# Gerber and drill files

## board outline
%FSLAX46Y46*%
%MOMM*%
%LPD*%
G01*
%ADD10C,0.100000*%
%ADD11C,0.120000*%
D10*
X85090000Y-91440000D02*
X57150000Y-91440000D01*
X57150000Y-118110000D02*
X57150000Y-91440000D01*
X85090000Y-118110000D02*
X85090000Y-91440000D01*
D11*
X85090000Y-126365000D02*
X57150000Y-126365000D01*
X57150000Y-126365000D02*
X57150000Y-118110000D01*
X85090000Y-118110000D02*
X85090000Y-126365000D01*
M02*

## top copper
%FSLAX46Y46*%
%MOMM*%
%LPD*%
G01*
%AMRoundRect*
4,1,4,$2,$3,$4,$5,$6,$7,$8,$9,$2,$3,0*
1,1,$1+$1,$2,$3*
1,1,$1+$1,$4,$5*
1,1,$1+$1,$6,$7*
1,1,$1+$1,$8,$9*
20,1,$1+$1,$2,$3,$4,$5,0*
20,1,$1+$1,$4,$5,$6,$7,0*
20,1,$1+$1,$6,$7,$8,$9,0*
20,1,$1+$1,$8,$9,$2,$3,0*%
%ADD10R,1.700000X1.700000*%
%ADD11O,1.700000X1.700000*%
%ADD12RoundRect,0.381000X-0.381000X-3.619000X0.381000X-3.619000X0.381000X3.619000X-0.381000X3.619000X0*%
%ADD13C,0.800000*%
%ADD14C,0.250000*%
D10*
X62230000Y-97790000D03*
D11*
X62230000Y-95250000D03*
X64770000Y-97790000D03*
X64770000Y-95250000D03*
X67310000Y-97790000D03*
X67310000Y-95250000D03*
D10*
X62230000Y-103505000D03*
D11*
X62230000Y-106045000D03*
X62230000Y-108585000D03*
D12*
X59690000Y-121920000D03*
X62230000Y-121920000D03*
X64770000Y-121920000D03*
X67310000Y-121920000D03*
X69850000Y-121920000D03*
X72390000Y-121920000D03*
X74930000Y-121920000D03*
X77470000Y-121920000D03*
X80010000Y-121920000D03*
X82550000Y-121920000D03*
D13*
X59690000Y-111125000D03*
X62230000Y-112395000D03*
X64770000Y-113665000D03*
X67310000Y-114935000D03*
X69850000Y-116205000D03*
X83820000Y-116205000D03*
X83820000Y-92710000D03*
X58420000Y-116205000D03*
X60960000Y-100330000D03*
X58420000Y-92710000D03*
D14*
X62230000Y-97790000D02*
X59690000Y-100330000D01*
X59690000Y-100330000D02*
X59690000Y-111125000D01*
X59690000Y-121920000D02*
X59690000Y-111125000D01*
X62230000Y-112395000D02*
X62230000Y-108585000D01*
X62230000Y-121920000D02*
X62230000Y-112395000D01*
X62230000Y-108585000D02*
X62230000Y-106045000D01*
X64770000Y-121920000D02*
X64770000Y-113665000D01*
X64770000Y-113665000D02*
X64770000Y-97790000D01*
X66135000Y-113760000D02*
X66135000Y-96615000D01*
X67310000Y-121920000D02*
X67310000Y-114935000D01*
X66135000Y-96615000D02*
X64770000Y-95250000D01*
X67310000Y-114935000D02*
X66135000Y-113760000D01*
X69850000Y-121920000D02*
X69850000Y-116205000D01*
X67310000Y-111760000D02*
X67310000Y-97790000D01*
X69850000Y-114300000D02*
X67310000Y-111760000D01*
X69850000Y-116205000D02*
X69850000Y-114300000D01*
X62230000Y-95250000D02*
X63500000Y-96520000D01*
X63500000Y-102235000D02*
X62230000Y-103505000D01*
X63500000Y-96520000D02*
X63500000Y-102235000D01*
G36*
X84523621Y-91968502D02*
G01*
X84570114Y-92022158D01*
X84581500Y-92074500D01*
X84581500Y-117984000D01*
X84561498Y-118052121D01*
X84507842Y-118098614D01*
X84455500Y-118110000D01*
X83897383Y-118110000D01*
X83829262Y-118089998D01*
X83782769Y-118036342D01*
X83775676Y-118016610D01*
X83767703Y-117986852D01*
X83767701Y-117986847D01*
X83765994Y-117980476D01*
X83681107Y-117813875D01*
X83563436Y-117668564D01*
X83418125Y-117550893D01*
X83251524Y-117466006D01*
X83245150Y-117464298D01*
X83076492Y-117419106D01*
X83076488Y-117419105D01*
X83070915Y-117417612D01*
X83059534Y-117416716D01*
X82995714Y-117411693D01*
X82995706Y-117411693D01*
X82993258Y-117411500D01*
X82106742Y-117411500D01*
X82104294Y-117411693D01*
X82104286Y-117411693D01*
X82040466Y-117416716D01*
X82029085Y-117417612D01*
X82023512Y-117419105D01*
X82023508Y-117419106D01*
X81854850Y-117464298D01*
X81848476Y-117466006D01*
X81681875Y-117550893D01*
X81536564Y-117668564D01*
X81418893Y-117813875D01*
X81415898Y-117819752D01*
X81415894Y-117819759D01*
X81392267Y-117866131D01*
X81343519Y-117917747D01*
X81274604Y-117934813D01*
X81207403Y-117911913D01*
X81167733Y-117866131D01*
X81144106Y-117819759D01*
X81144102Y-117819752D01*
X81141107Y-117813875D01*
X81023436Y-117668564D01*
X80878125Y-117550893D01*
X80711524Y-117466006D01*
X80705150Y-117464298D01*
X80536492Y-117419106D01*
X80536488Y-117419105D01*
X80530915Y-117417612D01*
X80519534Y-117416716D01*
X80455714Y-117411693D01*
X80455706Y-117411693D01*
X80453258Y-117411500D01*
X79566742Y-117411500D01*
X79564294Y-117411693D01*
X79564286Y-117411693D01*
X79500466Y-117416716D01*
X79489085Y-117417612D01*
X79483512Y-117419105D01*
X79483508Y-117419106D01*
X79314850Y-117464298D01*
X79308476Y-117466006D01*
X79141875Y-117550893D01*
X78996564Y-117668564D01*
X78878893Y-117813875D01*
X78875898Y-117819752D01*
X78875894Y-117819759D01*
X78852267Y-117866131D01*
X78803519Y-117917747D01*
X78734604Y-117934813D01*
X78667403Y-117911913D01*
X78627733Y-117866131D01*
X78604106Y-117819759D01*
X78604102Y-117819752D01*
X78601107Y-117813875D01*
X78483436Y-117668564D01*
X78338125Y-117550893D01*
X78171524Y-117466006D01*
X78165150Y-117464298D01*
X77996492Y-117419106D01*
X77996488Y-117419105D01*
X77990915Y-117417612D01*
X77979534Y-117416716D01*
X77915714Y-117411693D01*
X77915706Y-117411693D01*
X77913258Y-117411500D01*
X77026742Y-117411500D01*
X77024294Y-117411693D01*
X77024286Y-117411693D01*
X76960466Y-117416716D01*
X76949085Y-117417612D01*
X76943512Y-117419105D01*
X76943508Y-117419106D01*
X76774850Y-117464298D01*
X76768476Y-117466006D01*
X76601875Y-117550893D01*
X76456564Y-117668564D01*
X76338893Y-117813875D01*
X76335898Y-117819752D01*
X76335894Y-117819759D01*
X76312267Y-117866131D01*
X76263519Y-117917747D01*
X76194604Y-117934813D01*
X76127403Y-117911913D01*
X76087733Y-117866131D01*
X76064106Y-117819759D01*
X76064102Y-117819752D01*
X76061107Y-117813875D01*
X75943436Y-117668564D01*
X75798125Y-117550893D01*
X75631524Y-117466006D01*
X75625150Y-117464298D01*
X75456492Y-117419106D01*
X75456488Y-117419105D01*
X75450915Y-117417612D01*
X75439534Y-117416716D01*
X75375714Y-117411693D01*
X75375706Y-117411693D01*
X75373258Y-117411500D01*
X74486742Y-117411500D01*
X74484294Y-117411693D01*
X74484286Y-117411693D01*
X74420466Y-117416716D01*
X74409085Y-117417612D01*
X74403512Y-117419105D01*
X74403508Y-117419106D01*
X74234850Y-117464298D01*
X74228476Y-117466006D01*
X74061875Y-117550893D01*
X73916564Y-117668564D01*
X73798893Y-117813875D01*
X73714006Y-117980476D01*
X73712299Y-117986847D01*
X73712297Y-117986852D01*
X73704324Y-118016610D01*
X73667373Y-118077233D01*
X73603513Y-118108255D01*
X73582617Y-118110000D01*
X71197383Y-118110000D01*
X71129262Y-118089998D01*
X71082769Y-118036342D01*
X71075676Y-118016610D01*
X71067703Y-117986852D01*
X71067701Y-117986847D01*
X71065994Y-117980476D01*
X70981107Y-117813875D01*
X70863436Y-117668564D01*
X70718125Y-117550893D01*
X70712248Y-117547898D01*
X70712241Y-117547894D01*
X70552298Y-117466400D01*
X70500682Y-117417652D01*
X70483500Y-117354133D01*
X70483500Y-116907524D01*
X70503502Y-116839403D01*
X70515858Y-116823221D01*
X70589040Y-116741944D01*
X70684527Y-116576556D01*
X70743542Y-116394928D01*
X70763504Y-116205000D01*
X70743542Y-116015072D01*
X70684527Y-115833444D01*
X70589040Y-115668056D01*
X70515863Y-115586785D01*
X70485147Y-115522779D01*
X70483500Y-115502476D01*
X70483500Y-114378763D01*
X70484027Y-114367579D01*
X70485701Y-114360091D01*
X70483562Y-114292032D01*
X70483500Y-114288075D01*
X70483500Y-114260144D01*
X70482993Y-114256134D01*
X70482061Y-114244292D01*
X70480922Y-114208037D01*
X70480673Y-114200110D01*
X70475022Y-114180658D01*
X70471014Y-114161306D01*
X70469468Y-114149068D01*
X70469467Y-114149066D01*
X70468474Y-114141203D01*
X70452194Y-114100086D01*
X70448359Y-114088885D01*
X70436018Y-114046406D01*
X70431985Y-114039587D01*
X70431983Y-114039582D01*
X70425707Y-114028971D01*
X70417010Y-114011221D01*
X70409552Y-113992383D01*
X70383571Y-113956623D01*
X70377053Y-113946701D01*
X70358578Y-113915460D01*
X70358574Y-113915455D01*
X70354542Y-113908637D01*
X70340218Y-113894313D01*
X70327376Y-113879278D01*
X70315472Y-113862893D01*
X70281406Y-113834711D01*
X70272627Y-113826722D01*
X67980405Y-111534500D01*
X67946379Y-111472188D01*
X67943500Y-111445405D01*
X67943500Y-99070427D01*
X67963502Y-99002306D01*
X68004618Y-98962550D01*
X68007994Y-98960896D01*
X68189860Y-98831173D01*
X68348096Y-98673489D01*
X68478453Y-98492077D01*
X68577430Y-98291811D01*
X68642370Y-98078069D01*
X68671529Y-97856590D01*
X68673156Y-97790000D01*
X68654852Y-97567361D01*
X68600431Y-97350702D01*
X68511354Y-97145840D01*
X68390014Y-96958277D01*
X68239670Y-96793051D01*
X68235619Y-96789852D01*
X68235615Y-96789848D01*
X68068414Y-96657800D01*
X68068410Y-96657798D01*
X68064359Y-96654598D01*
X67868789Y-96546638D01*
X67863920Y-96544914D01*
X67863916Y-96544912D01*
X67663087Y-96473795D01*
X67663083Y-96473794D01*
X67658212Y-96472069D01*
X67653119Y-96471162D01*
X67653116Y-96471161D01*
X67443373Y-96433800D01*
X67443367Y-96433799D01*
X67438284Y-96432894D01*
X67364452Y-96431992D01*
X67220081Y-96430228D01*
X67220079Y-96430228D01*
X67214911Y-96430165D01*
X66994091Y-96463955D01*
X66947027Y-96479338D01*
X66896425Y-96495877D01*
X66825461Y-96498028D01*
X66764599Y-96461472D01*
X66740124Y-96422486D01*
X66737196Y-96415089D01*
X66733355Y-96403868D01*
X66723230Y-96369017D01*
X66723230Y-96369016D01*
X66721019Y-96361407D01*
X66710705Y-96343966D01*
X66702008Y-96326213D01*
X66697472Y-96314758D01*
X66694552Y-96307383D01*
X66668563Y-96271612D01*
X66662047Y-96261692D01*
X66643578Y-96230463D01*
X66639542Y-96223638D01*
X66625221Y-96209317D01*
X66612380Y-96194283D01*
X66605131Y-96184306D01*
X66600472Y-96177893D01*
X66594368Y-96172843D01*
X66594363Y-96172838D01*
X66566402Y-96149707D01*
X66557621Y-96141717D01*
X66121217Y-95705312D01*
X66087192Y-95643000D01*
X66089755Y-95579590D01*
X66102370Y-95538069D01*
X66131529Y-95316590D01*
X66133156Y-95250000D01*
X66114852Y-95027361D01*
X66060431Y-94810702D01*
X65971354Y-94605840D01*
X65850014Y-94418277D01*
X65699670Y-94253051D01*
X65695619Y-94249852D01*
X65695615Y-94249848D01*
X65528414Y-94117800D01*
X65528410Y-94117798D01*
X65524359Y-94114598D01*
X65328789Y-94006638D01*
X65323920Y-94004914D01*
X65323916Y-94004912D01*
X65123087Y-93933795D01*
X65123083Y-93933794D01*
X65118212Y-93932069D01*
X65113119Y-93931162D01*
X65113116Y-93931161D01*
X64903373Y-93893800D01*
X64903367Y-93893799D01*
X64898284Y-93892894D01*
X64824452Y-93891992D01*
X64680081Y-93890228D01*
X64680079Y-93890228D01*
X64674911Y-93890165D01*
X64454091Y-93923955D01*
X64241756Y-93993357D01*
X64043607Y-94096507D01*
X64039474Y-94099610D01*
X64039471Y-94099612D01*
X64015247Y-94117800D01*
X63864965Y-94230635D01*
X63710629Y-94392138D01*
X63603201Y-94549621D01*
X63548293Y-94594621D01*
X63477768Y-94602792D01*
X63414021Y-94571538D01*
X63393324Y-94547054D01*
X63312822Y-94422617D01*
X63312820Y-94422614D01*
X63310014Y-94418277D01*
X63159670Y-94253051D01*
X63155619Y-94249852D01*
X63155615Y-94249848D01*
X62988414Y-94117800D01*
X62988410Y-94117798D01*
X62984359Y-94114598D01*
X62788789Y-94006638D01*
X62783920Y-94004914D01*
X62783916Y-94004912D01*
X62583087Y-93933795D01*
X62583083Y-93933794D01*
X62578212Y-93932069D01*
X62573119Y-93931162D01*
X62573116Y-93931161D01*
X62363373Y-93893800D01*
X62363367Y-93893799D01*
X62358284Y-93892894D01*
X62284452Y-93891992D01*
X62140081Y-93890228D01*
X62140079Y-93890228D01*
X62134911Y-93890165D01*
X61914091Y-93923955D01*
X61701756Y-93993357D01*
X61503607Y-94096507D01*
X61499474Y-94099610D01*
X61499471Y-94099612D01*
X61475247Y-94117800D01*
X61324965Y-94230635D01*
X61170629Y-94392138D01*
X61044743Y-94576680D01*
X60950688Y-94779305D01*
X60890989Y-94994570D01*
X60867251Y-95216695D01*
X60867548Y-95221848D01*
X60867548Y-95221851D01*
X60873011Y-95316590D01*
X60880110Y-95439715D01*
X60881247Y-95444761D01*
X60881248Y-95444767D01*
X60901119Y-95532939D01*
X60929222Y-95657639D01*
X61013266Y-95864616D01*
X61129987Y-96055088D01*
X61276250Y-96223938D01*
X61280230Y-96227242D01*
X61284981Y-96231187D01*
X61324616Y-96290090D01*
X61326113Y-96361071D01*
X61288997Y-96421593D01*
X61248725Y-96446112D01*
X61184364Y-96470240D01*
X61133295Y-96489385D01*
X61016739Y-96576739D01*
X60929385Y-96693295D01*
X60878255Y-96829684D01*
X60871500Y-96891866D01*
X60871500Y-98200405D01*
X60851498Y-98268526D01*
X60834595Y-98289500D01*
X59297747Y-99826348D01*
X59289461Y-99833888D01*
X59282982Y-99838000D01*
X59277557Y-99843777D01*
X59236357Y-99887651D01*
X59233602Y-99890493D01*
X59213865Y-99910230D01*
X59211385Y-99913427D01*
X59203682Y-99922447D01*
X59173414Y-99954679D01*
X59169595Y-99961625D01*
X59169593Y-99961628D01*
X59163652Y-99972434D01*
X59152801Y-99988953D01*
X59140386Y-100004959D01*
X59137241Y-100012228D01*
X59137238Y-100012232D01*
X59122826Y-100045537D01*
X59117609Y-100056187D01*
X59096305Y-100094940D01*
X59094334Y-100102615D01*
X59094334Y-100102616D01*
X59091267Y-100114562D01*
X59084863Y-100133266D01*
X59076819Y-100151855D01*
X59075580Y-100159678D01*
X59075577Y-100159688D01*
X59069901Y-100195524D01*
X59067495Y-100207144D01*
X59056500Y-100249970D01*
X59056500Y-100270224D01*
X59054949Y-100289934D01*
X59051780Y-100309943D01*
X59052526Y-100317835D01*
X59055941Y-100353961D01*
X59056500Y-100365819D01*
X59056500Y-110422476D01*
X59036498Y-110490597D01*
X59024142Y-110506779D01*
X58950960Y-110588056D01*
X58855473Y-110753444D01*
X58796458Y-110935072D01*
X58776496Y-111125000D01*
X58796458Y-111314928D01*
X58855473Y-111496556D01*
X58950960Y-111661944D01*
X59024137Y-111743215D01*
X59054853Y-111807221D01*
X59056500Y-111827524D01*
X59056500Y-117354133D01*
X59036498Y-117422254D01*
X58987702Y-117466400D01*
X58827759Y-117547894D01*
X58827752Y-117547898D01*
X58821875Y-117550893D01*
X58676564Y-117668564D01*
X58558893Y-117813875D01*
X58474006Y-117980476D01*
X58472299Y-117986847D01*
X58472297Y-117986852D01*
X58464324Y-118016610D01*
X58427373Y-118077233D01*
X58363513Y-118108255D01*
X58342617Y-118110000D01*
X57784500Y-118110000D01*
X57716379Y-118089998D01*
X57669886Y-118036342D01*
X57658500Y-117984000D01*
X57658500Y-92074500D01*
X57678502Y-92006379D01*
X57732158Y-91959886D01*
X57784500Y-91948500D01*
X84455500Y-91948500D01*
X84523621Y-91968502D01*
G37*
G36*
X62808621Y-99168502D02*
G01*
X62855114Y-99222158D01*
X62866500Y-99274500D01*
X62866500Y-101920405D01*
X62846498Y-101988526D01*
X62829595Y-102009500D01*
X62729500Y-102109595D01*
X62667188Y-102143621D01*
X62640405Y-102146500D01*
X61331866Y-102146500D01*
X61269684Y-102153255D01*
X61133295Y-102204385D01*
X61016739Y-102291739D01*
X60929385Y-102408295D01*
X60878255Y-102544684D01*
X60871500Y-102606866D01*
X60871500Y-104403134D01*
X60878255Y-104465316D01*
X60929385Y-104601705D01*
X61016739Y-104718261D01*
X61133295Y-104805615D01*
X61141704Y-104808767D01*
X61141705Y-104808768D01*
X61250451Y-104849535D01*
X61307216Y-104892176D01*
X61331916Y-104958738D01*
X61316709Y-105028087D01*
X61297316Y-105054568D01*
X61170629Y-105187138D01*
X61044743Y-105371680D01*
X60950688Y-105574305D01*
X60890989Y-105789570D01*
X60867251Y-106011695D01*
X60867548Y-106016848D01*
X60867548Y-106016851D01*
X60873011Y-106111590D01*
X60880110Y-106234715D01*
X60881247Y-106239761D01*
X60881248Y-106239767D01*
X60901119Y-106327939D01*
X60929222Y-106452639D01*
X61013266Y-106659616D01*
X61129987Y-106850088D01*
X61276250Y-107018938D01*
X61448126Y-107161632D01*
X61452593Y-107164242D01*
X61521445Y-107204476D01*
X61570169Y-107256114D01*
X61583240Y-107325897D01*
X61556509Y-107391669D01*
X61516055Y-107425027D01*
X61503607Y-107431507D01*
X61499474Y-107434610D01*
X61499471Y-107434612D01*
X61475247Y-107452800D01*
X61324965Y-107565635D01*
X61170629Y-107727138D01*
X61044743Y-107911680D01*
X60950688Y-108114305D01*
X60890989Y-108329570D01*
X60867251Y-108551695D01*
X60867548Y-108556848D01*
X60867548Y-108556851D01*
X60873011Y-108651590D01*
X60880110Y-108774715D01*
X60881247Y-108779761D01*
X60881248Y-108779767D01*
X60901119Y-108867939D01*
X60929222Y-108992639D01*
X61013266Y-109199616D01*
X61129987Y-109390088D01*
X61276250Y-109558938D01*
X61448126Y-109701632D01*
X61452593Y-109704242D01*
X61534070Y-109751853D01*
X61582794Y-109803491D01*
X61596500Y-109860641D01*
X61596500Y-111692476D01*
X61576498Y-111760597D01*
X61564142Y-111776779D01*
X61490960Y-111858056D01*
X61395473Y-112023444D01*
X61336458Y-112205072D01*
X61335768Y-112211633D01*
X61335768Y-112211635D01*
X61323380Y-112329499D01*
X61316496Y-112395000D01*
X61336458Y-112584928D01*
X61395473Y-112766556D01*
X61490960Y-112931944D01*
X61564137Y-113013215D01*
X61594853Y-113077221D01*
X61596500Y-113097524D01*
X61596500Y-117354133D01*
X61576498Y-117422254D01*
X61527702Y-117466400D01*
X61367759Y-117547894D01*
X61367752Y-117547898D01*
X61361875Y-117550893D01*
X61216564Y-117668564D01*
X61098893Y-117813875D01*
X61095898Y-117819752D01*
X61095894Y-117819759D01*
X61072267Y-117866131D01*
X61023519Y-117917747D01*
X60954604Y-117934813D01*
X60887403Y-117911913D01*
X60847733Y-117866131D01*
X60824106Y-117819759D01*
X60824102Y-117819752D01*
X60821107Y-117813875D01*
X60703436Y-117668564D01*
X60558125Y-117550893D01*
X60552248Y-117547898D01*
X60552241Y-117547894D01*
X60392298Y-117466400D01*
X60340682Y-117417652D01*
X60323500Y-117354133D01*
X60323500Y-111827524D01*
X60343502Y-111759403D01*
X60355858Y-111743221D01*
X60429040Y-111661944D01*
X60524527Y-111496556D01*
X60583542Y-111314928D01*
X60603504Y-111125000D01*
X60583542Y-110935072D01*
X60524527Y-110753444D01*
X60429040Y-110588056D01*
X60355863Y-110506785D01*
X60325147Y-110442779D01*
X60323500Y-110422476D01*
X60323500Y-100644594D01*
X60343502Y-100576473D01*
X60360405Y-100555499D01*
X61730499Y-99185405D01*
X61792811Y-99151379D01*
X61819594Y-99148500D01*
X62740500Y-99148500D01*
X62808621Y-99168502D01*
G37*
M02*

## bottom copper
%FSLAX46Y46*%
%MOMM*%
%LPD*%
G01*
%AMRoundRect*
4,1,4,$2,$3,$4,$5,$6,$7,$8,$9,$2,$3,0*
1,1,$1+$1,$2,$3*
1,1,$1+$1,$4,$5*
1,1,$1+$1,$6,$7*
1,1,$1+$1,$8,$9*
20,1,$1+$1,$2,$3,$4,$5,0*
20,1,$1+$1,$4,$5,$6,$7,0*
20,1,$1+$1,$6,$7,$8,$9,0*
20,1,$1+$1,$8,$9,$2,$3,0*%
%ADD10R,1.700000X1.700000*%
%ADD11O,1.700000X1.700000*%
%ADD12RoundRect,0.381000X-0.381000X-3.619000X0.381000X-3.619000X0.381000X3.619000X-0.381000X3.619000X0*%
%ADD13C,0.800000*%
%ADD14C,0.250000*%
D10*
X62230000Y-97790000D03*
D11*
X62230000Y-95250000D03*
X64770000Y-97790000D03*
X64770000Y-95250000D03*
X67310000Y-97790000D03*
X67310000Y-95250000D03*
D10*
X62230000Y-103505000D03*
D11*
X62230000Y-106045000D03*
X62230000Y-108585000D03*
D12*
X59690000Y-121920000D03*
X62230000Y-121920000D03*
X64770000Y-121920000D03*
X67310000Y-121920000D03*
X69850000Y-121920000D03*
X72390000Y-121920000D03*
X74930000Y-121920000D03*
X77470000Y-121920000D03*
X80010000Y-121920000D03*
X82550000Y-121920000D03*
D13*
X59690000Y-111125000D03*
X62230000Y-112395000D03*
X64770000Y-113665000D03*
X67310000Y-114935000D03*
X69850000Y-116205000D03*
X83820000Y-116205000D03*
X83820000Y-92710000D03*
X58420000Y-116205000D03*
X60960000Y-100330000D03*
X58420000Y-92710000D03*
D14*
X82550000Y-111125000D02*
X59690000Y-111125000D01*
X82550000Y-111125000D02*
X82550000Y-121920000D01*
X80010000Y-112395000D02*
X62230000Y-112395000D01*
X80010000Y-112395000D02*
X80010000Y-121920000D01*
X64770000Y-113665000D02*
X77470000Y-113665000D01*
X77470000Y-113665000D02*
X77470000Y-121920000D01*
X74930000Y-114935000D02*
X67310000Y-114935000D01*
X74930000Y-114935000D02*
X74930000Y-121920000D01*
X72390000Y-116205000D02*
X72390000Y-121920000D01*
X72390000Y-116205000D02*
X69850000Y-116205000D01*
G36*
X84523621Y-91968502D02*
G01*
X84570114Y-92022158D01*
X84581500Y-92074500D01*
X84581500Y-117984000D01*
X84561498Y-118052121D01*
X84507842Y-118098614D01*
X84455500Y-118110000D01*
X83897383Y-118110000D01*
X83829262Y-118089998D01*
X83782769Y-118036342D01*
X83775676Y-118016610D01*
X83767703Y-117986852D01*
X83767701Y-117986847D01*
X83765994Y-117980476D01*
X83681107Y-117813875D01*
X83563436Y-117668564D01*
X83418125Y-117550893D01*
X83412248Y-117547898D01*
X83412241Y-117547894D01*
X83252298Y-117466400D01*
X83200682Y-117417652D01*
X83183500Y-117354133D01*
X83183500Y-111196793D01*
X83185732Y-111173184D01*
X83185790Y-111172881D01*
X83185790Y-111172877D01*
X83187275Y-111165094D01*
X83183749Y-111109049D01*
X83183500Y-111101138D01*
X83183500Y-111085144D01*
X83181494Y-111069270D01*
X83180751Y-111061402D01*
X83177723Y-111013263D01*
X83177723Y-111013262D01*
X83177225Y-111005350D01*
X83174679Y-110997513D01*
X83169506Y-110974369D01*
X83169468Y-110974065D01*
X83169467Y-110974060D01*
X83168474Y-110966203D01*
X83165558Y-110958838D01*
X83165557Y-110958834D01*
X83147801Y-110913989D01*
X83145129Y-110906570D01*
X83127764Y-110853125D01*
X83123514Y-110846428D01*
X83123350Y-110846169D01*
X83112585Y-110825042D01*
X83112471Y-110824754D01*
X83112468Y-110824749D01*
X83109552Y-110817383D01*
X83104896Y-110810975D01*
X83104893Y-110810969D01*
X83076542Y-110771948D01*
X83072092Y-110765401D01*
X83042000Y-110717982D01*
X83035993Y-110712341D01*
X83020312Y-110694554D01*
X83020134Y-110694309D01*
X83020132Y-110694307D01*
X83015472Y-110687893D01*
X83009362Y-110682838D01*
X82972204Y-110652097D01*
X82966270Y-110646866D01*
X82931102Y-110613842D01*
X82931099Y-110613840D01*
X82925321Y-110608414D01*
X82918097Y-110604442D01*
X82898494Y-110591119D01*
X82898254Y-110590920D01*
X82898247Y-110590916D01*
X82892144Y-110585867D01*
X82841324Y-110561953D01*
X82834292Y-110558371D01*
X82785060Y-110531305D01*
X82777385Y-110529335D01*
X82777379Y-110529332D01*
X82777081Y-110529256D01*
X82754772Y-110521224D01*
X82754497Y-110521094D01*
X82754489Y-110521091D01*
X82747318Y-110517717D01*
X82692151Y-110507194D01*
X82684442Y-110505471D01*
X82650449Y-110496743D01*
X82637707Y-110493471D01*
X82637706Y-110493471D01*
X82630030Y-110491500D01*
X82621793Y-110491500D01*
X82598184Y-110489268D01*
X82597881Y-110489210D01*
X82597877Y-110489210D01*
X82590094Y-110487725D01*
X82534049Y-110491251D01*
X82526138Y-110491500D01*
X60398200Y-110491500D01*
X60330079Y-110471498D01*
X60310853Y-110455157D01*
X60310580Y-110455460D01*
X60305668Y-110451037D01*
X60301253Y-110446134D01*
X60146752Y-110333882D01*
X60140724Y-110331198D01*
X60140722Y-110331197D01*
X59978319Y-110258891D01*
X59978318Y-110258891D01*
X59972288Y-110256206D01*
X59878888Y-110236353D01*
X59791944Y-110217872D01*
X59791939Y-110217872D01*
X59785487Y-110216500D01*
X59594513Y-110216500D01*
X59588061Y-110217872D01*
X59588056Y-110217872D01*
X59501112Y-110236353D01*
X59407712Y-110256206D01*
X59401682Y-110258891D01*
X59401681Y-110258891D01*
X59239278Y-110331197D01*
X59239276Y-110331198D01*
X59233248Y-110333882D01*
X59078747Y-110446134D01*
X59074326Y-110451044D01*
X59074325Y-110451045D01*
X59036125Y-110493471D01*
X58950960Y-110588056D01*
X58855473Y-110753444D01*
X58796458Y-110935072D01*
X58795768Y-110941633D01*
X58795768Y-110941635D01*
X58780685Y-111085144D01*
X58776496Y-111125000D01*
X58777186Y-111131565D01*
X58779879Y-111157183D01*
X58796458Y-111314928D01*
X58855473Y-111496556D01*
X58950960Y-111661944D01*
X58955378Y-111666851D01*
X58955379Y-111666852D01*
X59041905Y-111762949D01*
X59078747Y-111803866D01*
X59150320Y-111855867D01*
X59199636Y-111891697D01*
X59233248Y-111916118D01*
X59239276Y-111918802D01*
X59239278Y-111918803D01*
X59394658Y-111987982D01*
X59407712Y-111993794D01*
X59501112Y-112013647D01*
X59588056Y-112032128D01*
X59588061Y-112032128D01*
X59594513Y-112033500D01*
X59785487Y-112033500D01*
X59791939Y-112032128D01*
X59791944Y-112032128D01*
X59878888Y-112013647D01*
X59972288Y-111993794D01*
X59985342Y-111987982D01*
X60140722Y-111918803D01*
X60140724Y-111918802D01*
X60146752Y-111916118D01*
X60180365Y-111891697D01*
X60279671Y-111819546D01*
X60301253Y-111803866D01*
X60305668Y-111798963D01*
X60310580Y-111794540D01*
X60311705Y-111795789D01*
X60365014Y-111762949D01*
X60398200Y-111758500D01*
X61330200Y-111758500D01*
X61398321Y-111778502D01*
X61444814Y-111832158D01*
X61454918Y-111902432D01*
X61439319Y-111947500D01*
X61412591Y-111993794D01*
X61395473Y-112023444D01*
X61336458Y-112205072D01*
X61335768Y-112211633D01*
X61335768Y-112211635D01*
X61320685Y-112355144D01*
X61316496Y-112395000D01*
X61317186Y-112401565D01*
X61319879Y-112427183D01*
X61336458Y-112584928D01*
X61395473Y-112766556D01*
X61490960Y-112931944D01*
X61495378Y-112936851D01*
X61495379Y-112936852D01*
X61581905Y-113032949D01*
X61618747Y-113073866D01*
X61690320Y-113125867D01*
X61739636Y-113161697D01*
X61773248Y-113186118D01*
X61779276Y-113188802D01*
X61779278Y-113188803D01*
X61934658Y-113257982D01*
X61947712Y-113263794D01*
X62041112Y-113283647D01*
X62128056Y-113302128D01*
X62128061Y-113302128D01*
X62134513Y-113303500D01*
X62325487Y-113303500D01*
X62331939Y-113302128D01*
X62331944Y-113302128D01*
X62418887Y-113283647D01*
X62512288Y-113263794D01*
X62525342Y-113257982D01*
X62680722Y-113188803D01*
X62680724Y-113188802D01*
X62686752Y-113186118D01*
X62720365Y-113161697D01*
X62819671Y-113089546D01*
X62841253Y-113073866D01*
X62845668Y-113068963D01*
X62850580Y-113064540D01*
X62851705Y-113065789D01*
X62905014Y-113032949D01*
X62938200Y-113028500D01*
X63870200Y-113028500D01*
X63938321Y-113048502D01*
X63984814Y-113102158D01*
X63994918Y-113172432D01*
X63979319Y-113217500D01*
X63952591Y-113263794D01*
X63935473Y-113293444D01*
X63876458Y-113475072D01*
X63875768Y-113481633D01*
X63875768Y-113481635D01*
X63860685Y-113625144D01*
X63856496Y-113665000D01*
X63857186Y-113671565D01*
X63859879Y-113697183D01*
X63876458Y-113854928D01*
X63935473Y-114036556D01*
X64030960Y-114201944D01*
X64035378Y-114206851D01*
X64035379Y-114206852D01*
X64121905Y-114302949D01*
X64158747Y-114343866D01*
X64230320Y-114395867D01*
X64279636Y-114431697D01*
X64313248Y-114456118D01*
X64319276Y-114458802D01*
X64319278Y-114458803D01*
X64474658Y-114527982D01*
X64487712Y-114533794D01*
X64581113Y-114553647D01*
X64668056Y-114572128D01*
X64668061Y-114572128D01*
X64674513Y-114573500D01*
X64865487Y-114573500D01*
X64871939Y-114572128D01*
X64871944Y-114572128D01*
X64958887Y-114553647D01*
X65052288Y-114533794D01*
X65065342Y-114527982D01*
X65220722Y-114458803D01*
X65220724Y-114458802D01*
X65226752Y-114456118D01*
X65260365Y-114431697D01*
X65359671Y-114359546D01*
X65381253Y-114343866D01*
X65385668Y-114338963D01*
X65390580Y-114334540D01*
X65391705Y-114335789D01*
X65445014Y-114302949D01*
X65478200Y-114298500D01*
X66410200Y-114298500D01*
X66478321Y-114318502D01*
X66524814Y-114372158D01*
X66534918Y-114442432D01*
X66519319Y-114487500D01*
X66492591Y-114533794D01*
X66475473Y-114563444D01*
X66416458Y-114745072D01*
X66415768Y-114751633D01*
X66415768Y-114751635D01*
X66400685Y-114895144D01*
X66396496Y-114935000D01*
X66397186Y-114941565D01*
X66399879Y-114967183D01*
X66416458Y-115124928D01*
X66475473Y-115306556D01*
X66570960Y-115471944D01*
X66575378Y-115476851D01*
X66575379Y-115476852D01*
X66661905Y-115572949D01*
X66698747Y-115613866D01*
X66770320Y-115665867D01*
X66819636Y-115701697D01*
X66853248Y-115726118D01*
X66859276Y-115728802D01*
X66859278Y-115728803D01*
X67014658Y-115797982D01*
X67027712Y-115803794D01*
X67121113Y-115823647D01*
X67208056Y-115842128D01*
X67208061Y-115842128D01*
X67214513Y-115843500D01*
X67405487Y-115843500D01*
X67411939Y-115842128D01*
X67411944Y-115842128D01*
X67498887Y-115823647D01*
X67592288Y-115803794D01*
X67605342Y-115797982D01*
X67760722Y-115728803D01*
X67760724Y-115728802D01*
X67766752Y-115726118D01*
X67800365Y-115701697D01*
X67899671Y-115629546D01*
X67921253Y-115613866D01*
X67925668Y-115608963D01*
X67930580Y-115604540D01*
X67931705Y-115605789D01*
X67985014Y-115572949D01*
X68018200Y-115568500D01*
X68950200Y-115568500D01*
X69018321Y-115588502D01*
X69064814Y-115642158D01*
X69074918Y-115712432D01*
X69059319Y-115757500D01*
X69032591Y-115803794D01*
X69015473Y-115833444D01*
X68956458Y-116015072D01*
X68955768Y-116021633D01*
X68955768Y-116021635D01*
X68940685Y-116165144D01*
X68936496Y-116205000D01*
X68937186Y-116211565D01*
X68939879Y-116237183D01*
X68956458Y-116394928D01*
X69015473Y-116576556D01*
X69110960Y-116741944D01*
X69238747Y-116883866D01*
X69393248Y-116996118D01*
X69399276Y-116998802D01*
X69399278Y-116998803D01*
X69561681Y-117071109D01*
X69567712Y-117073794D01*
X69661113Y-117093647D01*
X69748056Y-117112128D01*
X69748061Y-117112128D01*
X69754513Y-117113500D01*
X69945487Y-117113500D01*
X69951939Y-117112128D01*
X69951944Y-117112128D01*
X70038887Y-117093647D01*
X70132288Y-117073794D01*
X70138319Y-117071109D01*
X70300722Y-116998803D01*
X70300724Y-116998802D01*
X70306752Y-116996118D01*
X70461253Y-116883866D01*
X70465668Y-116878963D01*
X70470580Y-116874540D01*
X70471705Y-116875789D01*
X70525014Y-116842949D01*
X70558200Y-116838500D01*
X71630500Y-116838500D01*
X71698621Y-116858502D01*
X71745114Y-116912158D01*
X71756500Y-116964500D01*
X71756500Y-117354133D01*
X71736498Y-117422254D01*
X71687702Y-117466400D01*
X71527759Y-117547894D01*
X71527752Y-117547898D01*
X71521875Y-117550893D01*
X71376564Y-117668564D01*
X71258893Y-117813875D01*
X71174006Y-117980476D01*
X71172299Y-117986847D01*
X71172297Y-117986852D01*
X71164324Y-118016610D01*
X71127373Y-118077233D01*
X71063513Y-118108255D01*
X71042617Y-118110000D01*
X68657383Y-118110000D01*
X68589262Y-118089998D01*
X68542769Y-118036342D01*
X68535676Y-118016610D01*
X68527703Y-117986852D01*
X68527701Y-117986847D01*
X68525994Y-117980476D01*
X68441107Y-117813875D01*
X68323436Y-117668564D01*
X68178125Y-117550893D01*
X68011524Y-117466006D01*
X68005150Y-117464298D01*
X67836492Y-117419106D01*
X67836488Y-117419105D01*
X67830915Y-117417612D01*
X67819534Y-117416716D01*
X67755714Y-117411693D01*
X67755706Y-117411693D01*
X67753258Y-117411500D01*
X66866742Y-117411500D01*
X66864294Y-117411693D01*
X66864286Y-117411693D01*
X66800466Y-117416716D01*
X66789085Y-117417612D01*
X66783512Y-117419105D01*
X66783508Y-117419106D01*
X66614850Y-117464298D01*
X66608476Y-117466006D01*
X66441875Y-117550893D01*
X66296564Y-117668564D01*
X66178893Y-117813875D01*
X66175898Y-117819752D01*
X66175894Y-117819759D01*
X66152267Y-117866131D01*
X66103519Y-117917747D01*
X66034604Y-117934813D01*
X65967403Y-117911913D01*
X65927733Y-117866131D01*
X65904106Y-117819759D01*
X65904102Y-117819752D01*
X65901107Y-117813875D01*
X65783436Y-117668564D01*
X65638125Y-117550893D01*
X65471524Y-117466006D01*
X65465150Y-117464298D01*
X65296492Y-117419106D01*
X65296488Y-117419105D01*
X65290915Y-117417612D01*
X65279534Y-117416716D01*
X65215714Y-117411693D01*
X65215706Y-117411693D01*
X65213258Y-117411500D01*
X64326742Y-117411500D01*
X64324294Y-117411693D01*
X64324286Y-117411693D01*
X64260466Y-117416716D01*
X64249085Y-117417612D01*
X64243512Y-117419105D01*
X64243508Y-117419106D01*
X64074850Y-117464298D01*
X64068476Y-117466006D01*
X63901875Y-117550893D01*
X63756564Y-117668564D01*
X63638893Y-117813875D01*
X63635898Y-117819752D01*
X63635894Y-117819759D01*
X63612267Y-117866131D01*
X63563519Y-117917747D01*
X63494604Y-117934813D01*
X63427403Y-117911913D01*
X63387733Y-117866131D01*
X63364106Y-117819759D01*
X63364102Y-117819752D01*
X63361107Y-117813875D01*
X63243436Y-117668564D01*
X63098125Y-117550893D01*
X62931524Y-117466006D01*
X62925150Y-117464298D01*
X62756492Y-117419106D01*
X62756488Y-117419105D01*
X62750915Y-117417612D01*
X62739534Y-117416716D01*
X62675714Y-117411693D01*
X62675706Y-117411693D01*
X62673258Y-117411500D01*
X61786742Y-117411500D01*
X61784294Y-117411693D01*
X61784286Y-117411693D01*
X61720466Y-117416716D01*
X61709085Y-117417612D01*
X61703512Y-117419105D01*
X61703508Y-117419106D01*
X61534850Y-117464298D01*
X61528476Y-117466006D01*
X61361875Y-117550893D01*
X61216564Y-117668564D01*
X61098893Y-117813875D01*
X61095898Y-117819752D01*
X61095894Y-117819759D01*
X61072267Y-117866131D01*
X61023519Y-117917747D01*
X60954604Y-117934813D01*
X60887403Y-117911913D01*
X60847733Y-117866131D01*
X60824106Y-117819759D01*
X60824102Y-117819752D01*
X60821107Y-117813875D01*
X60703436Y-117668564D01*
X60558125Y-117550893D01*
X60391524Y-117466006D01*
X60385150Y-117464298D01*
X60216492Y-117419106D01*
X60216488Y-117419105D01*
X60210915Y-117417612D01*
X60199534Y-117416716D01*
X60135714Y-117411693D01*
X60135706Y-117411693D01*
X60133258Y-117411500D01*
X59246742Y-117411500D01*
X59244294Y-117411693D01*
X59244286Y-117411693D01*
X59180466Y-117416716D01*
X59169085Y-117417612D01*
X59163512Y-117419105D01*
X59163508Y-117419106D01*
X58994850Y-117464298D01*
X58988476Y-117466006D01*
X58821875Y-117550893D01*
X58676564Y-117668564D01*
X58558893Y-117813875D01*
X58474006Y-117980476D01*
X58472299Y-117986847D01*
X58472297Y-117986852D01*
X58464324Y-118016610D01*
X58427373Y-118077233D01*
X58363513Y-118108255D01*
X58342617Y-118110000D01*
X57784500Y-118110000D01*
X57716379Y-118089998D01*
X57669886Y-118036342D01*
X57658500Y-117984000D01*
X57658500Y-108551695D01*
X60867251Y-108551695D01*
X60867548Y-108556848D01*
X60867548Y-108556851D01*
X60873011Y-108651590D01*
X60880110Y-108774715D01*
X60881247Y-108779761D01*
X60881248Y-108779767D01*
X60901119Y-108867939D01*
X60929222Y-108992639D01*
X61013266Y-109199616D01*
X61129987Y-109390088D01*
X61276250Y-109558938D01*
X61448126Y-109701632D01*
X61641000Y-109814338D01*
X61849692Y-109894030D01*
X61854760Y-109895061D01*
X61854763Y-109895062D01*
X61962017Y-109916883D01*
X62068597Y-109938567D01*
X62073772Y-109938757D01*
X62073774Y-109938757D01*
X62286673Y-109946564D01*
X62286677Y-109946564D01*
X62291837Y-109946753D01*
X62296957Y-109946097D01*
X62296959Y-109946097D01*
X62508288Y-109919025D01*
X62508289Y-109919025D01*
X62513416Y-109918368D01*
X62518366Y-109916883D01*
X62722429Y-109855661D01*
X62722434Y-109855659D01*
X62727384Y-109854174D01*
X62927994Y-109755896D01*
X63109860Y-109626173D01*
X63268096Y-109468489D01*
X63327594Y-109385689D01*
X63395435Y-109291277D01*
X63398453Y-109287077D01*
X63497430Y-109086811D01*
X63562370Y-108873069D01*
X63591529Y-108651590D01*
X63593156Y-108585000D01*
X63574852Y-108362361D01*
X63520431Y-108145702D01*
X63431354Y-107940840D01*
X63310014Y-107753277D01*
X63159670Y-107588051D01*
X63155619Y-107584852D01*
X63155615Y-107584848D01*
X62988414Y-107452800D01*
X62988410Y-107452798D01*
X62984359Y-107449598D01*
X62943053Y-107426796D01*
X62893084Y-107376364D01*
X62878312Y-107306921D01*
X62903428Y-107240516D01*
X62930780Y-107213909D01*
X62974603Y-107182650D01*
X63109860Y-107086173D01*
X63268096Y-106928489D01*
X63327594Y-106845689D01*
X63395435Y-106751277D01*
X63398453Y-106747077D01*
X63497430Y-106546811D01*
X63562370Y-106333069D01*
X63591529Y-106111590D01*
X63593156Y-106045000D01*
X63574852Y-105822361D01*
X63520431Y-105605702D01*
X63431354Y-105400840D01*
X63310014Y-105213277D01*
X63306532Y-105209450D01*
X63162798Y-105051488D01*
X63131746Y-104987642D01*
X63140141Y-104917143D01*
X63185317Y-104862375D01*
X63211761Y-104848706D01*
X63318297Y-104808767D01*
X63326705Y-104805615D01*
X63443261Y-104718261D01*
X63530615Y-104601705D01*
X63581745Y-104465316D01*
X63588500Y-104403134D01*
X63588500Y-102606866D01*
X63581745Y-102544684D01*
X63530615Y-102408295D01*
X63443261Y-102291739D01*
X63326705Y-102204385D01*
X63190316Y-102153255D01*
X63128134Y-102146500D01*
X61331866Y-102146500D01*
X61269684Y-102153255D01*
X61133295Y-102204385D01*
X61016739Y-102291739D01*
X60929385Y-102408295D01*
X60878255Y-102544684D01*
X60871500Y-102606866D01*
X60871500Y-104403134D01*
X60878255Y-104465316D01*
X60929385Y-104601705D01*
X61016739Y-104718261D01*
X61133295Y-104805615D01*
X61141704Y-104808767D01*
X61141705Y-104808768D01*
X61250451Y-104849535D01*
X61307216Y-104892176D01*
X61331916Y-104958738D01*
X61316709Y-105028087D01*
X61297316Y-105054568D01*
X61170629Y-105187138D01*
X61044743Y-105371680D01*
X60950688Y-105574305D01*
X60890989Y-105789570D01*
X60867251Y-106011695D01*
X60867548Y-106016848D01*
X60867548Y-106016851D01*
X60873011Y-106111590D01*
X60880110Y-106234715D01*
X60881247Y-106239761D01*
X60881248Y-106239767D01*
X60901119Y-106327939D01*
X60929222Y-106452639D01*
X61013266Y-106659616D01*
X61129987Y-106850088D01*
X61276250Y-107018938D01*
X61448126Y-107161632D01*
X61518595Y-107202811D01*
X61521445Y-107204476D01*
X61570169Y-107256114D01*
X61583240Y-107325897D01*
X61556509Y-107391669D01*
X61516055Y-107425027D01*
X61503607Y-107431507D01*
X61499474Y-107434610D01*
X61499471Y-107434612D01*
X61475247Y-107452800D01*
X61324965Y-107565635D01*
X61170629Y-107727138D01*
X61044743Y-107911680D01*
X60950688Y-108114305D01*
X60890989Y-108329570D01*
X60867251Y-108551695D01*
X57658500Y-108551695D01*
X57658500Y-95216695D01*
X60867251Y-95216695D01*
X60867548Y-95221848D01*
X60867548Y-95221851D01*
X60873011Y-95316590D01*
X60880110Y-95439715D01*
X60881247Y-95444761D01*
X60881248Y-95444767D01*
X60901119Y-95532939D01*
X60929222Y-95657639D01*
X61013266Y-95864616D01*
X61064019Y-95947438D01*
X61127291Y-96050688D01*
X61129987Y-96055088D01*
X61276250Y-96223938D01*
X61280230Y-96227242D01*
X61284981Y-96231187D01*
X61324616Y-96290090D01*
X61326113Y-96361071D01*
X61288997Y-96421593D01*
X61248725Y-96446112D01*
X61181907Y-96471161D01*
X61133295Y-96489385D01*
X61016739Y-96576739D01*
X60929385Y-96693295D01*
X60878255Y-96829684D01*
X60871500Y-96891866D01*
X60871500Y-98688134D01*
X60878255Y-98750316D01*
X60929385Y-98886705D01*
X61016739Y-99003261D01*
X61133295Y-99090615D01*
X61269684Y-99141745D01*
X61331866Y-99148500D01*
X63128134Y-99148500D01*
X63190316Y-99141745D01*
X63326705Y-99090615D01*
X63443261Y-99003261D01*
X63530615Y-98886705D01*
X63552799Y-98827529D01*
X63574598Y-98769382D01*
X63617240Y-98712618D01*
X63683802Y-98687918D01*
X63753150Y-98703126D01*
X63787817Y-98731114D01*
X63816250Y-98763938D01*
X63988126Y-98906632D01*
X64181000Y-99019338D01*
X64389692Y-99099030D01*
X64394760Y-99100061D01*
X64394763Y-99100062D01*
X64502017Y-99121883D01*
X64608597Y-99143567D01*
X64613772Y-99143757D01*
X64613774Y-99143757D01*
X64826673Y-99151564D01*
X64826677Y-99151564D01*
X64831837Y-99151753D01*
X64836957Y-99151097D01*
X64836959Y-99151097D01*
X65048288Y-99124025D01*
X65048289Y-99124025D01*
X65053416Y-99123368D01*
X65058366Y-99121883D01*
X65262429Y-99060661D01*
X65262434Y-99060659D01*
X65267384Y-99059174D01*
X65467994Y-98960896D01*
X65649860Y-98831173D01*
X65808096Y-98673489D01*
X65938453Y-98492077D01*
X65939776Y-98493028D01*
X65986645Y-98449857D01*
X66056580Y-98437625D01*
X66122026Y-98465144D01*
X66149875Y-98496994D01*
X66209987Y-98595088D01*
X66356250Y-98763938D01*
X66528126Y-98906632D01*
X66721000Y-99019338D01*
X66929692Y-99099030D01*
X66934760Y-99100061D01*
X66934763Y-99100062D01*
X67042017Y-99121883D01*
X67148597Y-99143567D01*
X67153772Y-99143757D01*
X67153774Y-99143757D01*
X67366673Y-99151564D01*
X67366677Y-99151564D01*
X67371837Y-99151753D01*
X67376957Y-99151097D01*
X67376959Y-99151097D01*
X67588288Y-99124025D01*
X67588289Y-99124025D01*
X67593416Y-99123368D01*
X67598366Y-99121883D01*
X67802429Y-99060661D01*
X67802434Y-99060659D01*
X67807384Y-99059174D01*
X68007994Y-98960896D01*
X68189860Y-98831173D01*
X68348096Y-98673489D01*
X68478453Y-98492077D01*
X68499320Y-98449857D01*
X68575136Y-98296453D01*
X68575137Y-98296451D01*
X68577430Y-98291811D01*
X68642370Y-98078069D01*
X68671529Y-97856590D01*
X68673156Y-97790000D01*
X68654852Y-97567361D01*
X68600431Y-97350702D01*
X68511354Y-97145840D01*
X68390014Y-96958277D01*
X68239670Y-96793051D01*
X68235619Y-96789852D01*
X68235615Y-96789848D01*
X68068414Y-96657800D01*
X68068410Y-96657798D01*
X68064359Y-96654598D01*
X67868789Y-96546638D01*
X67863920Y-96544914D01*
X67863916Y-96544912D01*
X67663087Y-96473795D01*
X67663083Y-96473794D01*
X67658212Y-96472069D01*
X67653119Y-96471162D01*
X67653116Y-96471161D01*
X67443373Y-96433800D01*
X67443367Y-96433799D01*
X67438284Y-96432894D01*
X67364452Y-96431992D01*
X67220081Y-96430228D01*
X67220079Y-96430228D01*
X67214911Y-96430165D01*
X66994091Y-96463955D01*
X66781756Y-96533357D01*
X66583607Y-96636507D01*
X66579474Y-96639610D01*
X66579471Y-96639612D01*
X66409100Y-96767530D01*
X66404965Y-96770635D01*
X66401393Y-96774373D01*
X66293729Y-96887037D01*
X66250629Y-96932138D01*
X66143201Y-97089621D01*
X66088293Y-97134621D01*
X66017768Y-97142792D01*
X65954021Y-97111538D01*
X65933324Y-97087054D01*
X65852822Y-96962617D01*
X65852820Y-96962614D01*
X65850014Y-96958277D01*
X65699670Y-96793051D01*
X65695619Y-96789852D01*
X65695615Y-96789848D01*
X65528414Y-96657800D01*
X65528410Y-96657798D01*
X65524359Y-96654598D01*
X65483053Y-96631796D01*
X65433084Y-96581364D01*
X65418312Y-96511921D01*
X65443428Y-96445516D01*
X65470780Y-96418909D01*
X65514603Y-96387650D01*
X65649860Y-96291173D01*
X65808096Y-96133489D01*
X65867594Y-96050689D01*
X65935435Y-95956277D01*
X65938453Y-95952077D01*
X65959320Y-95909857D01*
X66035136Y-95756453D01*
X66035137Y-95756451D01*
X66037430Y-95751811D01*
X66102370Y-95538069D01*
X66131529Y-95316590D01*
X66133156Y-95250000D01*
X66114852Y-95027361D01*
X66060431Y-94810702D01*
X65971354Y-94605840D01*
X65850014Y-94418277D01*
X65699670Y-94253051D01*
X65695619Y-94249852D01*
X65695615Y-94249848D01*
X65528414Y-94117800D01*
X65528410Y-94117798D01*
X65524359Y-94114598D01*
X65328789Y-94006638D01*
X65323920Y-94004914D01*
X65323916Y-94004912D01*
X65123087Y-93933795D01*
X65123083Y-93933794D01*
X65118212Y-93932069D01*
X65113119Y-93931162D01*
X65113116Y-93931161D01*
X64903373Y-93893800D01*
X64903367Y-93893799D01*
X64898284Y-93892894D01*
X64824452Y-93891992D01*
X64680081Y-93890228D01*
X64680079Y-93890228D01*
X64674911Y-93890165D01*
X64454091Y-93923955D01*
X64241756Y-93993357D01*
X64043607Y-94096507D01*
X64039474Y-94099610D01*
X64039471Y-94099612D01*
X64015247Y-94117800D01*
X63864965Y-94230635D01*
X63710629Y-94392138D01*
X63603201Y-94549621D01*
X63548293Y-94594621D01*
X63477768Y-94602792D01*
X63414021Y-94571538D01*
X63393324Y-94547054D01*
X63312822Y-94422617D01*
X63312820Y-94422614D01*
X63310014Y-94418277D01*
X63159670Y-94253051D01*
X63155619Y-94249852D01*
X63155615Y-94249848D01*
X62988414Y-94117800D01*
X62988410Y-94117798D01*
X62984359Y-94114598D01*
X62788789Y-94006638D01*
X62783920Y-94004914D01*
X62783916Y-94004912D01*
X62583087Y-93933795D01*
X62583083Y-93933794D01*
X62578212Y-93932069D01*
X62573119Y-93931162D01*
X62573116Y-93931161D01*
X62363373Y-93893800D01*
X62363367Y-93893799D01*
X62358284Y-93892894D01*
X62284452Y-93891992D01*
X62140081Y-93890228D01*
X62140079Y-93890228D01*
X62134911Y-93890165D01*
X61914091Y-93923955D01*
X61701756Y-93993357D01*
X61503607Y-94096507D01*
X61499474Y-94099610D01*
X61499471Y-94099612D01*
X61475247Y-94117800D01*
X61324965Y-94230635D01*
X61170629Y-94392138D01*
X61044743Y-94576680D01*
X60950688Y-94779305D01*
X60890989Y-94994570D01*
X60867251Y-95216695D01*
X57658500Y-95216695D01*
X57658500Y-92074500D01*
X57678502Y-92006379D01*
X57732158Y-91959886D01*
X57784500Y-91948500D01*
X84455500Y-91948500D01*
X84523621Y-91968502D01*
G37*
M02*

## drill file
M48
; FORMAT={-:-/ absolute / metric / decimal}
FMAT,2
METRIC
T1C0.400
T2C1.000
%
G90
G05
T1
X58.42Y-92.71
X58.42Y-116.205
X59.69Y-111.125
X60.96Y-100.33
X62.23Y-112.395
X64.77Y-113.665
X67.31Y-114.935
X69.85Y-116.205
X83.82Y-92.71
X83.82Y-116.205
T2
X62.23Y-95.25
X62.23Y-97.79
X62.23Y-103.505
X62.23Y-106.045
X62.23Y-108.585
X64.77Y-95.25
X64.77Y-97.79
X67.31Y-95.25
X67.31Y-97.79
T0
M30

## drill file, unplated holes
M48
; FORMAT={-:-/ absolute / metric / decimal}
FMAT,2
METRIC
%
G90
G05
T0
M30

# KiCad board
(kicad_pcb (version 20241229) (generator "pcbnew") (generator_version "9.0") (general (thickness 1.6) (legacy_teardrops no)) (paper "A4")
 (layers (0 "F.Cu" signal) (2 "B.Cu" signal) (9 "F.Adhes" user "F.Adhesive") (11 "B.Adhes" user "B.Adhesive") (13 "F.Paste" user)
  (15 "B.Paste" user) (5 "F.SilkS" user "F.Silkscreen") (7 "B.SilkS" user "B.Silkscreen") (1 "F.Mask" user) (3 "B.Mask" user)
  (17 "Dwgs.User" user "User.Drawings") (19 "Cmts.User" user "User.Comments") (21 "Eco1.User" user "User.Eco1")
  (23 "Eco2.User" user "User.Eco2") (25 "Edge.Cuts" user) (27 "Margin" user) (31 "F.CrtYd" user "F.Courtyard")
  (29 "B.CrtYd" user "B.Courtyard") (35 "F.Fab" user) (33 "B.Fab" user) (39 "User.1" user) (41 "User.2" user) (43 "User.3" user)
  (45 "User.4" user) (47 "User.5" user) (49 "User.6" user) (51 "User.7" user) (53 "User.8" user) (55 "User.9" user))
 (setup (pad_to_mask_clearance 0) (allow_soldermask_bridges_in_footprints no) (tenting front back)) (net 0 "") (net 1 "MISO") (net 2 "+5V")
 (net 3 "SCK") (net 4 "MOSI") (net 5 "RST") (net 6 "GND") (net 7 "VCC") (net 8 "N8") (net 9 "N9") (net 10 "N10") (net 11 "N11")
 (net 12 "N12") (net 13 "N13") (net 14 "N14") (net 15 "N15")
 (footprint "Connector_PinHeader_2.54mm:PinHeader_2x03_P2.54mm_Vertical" (layer "F.Cu") (at 62.23 97.79 90)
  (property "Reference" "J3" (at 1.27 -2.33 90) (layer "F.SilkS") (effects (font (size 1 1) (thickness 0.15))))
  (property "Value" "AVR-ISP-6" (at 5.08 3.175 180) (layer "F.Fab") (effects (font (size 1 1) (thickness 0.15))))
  (pad "1" thru_hole rect (at 0 0 90) (size 1.7 1.7) (drill 1) (layers "*.Cu" "*.Mask") (remove_unused_layers no) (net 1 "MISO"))
  (pad "2" thru_hole oval (at 2.54 0 90) (size 1.7 1.7) (drill 1) (layers "*.Cu" "*.Mask") (remove_unused_layers no) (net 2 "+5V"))
  (pad "3" thru_hole oval (at 0 2.54 90) (size 1.7 1.7) (drill 1) (layers "*.Cu" "*.Mask") (remove_unused_layers no) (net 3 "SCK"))
  (pad "4" thru_hole oval (at 2.54 2.54 90) (size 1.7 1.7) (drill 1) (layers "*.Cu" "*.Mask") (remove_unused_layers no) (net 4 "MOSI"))
  (pad "5" thru_hole oval (at 0 5.08 90) (size 1.7 1.7) (drill 1) (layers "*.Cu" "*.Mask") (remove_unused_layers no) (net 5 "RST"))
  (pad "6" thru_hole oval (at 2.54 5.08 90) (size 1.7 1.7) (drill 1) (layers "*.Cu" "*.Mask") (remove_unused_layers no) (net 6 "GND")))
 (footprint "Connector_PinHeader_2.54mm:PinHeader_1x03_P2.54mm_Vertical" (layer "F.Cu") (at 62.23 103.505)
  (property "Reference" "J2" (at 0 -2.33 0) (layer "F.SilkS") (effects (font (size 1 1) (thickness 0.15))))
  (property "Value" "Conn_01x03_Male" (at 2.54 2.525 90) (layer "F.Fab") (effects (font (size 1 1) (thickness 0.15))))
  (pad "1" thru_hole rect (at 0 0) (size 1.7 1.7) (drill 1) (layers "*.Cu" "*.Mask") (remove_unused_layers no) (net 2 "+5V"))
  (pad "2" thru_hole oval (at 0 2.54) (size 1.7 1.7) (drill 1) (layers "*.Cu" "*.Mask") (remove_unused_layers no) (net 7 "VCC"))
  (pad "3" thru_hole oval (at 0 5.08) (size 1.7 1.7) (drill 1) (layers "*.Cu" "*.Mask") (remove_unused_layers no) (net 7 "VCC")))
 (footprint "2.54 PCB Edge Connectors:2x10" (layer "F.Cu") (at 57.15 125.73)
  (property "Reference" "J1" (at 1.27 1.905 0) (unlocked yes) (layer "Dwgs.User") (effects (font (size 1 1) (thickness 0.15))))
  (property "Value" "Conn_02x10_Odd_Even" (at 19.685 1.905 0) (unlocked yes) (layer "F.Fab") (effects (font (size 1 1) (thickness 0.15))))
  (fp_line (start 0 0.635) (end 0 -7.62) (stroke (width 0.12) (type solid)) (layer "Edge.Cuts"))
  (fp_line (start 27.94 -7.62) (end 27.94 0.635) (stroke (width 0.12) (type solid)) (layer "Edge.Cuts"))
  (fp_line (start 27.94 0.635) (end 0 0.635) (stroke (width 0.12) (type solid)) (layer "Edge.Cuts"))
  (pad "1" connect roundrect (at 2.54 -3.81) (size 1.524 8) (layers "F.Cu" "F.Mask") (roundrect_rratio 0.25) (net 1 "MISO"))
  (pad "2" connect roundrect (at 2.54 -3.81) (size 1.524 8) (layers "B.Cu" "B.Mask") (roundrect_rratio 0.25) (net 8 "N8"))
  (pad "3" connect roundrect (at 5.08 -3.81) (size 1.524 8) (layers "F.Cu" "F.Mask") (roundrect_rratio 0.25) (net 7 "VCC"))
  (pad "4" connect roundrect (at 5.08 -3.81) (size 1.524 8) (layers "B.Cu" "B.Mask") (roundrect_rratio 0.25) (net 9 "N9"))
  (pad "5" connect roundrect (at 7.62 -3.81) (size 1.524 8) (layers "F.Cu" "F.Mask") (roundrect_rratio 0.25) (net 3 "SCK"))
  (pad "6" connect roundrect (at 7.62 -3.81) (size 1.524 8) (layers "B.Cu" "B.Mask") (roundrect_rratio 0.25) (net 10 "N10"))
  (pad "7" connect roundrect (at 10.16 -3.81) (size 1.524 8) (layers "F.Cu" "F.Mask") (roundrect_rratio 0.25) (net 4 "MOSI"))
  (pad "8" connect roundrect (at 10.16 -3.81) (size 1.524 8) (layers "B.Cu" "B.Mask") (roundrect_rratio 0.25) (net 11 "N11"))
  (pad "9" connect roundrect (at 12.7 -3.81) (size 1.524 8) (layers "F.Cu" "F.Mask") (roundrect_rratio 0.25) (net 5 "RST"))
  (pad "10" connect roundrect (at 12.7 -3.81) (size 1.524 8) (layers "B.Cu" "B.Mask") (roundrect_rratio 0.25) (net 6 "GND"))
  (pad "11" connect roundrect (at 15.24 -3.81) (size 1.524 8) (layers "F.Cu" "F.Mask") (roundrect_rratio 0.25) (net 6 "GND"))
  (pad "12" connect roundrect (at 15.24 -3.81) (size 1.524 8) (layers "B.Cu" "B.Mask") (roundrect_rratio 0.25) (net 5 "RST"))
  (pad "13" connect roundrect (at 17.78 -3.81) (size 1.524 8) (layers "F.Cu" "F.Mask") (roundrect_rratio 0.25) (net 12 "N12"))
  (pad "14" connect roundrect (at 17.78 -3.81) (size 1.524 8) (layers "B.Cu" "B.Mask") (roundrect_rratio 0.25) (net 4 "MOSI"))
  (pad "15" connect roundrect (at 20.32 -3.81) (size 1.524 8) (layers "F.Cu" "F.Mask") (roundrect_rratio 0.25) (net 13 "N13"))
  (pad "16" connect roundrect (at 20.32 -3.81) (size 1.524 8) (layers "B.Cu" "B.Mask") (roundrect_rratio 0.25) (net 3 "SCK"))
  (pad "17" connect roundrect (at 22.86 -3.81) (size 1.524 8) (layers "F.Cu" "F.Mask") (roundrect_rratio 0.25) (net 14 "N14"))
  (pad "18" connect roundrect (at 22.86 -3.81) (size 1.524 8) (layers "B.Cu" "B.Mask") (roundrect_rratio 0.25) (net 7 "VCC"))
  (pad "19" connect roundrect (at 25.4 -3.81) (size 1.524 8) (layers "F.Cu" "F.Mask") (roundrect_rratio 0.25) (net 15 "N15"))
  (pad "20" connect roundrect (at 25.4 -3.81) (size 1.524 8) (layers "B.Cu" "B.Mask") (roundrect_rratio 0.25) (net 1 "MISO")))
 (gr_line (start 85.09 91.44) (end 57.15 91.44) (stroke (width 0.1) (type solid)) (layer "Edge.Cuts"))
 (gr_line (start 57.15 118.11) (end 57.15 91.44) (stroke (width 0.1) (type solid)) (layer "Edge.Cuts"))
 (gr_line (start 85.09 118.11) (end 85.09 91.44) (stroke (width 0.1) (type solid)) (layer "Edge.Cuts"))
 (segment (start 62.23 97.79) (end 59.69 100.33) (width 0.25) (layer "F.Cu") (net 1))
 (segment (start 59.69 100.33) (end 59.69 111.125) (width 0.25) (layer "F.Cu") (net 1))
 (segment (start 59.69 121.92) (end 59.69 111.125) (width 0.25) (layer "F.Cu") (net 1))
 (via (at 59.69 111.125) (size 0.8) (drill 0.4) (layers "F.Cu" "B.Cu") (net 1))
 (segment (start 82.55 111.125) (end 59.69 111.125) (width 0.25) (layer "B.Cu") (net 1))
 (segment (start 82.55 111.125) (end 82.55 121.92) (width 0.25) (layer "B.Cu") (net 1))
 (segment (start 62.23 112.395) (end 62.23 108.585) (width 0.25) (layer "F.Cu") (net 7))
 (segment (start 62.23 121.92) (end 62.23 112.395) (width 0.25) (layer "F.Cu") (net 7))
 (segment (start 62.23 108.585) (end 62.23 106.045) (width 0.25) (layer "F.Cu") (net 7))
 (via (at 62.23 112.395) (size 0.8) (drill 0.4) (layers "F.Cu" "B.Cu") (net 7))
 (segment (start 80.01 112.395) (end 62.23 112.395) (width 0.25) (layer "B.Cu") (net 7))
 (segment (start 80.01 112.395) (end 80.01 121.92) (width 0.25) (layer "B.Cu") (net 7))
 (segment (start 64.77 121.92) (end 64.77 113.665) (width 0.25) (layer "F.Cu") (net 3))
 (segment (start 64.77 113.665) (end 64.77 97.79) (width 0.25) (layer "F.Cu") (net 3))
 (via (at 64.77 113.665) (size 0.8) (drill 0.4) (layers "F.Cu" "B.Cu") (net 3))
 (segment (start 64.77 113.665) (end 77.47 113.665) (width 0.25) (layer "B.Cu") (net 3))
 (segment (start 77.47 113.665) (end 77.47 121.92) (width 0.25) (layer "B.Cu") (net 3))
 (segment (start 66.135 113.76) (end 66.135 96.615) (width 0.25) (layer "F.Cu") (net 4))
 (segment (start 67.31 121.92) (end 67.31 114.935) (width 0.25) (layer "F.Cu") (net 4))
 (segment (start 66.135 96.615) (end 64.77 95.25) (width 0.25) (layer "F.Cu") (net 4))
 (segment (start 67.31 114.935) (end 66.135 113.76) (width 0.25) (layer "F.Cu") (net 4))
 (via (at 67.31 114.935) (size 0.8) (drill 0.4) (layers "F.Cu" "B.Cu") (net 4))
 (segment (start 74.93 114.935) (end 67.31 114.935) (width 0.25) (layer "B.Cu") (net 4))
 (segment (start 74.93 114.935) (end 74.93 121.92) (width 0.25) (layer "B.Cu") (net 4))
 (segment (start 69.85 121.92) (end 69.85 116.205) (width 0.25) (layer "F.Cu") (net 5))
 (segment (start 67.31 111.76) (end 67.31 97.79) (width 0.25) (layer "F.Cu") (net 5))
 (segment (start 69.85 114.3) (end 67.31 111.76) (width 0.25) (layer "F.Cu") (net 5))
 (segment (start 69.85 116.205) (end 69.85 114.3) (width 0.25) (layer "F.Cu") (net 5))
 (via (at 69.85 116.205) (size 0.8) (drill 0.4) (layers "F.Cu" "B.Cu") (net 5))
 (segment (start 72.39 116.205) (end 72.39 121.92) (width 0.25) (layer "B.Cu") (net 5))
 (segment (start 72.39 116.205) (end 69.85 116.205) (width 0.25) (layer "B.Cu") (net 5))
 (via (at 83.82 116.205) (size 0.8) (drill 0.4) (layers "F.Cu" "B.Cu") (free yes) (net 6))
 (via (at 83.82 92.71) (size 0.8) (drill 0.4) (layers "F.Cu" "B.Cu") (free yes) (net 6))
 (via (at 58.42 116.205) (size 0.8) (drill 0.4) (layers "F.Cu" "B.Cu") (free yes) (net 6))
 (via (at 60.96 100.33) (size 0.8) (drill 0.4) (layers "F.Cu" "B.Cu") (free yes) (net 6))
 (via (at 58.42 92.71) (size 0.8) (drill 0.4) (layers "F.Cu" "B.Cu") (free yes) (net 6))
 (segment (start 62.23 95.25) (end 63.5 96.52) (width 0.25) (layer "F.Cu") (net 2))
 (segment (start 63.5 102.235) (end 62.23 103.505) (width 0.25) (layer "F.Cu") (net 2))
 (segment (start 63.5 96.52) (end 63.5 102.235) (width 0.25) (layer "F.Cu") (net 2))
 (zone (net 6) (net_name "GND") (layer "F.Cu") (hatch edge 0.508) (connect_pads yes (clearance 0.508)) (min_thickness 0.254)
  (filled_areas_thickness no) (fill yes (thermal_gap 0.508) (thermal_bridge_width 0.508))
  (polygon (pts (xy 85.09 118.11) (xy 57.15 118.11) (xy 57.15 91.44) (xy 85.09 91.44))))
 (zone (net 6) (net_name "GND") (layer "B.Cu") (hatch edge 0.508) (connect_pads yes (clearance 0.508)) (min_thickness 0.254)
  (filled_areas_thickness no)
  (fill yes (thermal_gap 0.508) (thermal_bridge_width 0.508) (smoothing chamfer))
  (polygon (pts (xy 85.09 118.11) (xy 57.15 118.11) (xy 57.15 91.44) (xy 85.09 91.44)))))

